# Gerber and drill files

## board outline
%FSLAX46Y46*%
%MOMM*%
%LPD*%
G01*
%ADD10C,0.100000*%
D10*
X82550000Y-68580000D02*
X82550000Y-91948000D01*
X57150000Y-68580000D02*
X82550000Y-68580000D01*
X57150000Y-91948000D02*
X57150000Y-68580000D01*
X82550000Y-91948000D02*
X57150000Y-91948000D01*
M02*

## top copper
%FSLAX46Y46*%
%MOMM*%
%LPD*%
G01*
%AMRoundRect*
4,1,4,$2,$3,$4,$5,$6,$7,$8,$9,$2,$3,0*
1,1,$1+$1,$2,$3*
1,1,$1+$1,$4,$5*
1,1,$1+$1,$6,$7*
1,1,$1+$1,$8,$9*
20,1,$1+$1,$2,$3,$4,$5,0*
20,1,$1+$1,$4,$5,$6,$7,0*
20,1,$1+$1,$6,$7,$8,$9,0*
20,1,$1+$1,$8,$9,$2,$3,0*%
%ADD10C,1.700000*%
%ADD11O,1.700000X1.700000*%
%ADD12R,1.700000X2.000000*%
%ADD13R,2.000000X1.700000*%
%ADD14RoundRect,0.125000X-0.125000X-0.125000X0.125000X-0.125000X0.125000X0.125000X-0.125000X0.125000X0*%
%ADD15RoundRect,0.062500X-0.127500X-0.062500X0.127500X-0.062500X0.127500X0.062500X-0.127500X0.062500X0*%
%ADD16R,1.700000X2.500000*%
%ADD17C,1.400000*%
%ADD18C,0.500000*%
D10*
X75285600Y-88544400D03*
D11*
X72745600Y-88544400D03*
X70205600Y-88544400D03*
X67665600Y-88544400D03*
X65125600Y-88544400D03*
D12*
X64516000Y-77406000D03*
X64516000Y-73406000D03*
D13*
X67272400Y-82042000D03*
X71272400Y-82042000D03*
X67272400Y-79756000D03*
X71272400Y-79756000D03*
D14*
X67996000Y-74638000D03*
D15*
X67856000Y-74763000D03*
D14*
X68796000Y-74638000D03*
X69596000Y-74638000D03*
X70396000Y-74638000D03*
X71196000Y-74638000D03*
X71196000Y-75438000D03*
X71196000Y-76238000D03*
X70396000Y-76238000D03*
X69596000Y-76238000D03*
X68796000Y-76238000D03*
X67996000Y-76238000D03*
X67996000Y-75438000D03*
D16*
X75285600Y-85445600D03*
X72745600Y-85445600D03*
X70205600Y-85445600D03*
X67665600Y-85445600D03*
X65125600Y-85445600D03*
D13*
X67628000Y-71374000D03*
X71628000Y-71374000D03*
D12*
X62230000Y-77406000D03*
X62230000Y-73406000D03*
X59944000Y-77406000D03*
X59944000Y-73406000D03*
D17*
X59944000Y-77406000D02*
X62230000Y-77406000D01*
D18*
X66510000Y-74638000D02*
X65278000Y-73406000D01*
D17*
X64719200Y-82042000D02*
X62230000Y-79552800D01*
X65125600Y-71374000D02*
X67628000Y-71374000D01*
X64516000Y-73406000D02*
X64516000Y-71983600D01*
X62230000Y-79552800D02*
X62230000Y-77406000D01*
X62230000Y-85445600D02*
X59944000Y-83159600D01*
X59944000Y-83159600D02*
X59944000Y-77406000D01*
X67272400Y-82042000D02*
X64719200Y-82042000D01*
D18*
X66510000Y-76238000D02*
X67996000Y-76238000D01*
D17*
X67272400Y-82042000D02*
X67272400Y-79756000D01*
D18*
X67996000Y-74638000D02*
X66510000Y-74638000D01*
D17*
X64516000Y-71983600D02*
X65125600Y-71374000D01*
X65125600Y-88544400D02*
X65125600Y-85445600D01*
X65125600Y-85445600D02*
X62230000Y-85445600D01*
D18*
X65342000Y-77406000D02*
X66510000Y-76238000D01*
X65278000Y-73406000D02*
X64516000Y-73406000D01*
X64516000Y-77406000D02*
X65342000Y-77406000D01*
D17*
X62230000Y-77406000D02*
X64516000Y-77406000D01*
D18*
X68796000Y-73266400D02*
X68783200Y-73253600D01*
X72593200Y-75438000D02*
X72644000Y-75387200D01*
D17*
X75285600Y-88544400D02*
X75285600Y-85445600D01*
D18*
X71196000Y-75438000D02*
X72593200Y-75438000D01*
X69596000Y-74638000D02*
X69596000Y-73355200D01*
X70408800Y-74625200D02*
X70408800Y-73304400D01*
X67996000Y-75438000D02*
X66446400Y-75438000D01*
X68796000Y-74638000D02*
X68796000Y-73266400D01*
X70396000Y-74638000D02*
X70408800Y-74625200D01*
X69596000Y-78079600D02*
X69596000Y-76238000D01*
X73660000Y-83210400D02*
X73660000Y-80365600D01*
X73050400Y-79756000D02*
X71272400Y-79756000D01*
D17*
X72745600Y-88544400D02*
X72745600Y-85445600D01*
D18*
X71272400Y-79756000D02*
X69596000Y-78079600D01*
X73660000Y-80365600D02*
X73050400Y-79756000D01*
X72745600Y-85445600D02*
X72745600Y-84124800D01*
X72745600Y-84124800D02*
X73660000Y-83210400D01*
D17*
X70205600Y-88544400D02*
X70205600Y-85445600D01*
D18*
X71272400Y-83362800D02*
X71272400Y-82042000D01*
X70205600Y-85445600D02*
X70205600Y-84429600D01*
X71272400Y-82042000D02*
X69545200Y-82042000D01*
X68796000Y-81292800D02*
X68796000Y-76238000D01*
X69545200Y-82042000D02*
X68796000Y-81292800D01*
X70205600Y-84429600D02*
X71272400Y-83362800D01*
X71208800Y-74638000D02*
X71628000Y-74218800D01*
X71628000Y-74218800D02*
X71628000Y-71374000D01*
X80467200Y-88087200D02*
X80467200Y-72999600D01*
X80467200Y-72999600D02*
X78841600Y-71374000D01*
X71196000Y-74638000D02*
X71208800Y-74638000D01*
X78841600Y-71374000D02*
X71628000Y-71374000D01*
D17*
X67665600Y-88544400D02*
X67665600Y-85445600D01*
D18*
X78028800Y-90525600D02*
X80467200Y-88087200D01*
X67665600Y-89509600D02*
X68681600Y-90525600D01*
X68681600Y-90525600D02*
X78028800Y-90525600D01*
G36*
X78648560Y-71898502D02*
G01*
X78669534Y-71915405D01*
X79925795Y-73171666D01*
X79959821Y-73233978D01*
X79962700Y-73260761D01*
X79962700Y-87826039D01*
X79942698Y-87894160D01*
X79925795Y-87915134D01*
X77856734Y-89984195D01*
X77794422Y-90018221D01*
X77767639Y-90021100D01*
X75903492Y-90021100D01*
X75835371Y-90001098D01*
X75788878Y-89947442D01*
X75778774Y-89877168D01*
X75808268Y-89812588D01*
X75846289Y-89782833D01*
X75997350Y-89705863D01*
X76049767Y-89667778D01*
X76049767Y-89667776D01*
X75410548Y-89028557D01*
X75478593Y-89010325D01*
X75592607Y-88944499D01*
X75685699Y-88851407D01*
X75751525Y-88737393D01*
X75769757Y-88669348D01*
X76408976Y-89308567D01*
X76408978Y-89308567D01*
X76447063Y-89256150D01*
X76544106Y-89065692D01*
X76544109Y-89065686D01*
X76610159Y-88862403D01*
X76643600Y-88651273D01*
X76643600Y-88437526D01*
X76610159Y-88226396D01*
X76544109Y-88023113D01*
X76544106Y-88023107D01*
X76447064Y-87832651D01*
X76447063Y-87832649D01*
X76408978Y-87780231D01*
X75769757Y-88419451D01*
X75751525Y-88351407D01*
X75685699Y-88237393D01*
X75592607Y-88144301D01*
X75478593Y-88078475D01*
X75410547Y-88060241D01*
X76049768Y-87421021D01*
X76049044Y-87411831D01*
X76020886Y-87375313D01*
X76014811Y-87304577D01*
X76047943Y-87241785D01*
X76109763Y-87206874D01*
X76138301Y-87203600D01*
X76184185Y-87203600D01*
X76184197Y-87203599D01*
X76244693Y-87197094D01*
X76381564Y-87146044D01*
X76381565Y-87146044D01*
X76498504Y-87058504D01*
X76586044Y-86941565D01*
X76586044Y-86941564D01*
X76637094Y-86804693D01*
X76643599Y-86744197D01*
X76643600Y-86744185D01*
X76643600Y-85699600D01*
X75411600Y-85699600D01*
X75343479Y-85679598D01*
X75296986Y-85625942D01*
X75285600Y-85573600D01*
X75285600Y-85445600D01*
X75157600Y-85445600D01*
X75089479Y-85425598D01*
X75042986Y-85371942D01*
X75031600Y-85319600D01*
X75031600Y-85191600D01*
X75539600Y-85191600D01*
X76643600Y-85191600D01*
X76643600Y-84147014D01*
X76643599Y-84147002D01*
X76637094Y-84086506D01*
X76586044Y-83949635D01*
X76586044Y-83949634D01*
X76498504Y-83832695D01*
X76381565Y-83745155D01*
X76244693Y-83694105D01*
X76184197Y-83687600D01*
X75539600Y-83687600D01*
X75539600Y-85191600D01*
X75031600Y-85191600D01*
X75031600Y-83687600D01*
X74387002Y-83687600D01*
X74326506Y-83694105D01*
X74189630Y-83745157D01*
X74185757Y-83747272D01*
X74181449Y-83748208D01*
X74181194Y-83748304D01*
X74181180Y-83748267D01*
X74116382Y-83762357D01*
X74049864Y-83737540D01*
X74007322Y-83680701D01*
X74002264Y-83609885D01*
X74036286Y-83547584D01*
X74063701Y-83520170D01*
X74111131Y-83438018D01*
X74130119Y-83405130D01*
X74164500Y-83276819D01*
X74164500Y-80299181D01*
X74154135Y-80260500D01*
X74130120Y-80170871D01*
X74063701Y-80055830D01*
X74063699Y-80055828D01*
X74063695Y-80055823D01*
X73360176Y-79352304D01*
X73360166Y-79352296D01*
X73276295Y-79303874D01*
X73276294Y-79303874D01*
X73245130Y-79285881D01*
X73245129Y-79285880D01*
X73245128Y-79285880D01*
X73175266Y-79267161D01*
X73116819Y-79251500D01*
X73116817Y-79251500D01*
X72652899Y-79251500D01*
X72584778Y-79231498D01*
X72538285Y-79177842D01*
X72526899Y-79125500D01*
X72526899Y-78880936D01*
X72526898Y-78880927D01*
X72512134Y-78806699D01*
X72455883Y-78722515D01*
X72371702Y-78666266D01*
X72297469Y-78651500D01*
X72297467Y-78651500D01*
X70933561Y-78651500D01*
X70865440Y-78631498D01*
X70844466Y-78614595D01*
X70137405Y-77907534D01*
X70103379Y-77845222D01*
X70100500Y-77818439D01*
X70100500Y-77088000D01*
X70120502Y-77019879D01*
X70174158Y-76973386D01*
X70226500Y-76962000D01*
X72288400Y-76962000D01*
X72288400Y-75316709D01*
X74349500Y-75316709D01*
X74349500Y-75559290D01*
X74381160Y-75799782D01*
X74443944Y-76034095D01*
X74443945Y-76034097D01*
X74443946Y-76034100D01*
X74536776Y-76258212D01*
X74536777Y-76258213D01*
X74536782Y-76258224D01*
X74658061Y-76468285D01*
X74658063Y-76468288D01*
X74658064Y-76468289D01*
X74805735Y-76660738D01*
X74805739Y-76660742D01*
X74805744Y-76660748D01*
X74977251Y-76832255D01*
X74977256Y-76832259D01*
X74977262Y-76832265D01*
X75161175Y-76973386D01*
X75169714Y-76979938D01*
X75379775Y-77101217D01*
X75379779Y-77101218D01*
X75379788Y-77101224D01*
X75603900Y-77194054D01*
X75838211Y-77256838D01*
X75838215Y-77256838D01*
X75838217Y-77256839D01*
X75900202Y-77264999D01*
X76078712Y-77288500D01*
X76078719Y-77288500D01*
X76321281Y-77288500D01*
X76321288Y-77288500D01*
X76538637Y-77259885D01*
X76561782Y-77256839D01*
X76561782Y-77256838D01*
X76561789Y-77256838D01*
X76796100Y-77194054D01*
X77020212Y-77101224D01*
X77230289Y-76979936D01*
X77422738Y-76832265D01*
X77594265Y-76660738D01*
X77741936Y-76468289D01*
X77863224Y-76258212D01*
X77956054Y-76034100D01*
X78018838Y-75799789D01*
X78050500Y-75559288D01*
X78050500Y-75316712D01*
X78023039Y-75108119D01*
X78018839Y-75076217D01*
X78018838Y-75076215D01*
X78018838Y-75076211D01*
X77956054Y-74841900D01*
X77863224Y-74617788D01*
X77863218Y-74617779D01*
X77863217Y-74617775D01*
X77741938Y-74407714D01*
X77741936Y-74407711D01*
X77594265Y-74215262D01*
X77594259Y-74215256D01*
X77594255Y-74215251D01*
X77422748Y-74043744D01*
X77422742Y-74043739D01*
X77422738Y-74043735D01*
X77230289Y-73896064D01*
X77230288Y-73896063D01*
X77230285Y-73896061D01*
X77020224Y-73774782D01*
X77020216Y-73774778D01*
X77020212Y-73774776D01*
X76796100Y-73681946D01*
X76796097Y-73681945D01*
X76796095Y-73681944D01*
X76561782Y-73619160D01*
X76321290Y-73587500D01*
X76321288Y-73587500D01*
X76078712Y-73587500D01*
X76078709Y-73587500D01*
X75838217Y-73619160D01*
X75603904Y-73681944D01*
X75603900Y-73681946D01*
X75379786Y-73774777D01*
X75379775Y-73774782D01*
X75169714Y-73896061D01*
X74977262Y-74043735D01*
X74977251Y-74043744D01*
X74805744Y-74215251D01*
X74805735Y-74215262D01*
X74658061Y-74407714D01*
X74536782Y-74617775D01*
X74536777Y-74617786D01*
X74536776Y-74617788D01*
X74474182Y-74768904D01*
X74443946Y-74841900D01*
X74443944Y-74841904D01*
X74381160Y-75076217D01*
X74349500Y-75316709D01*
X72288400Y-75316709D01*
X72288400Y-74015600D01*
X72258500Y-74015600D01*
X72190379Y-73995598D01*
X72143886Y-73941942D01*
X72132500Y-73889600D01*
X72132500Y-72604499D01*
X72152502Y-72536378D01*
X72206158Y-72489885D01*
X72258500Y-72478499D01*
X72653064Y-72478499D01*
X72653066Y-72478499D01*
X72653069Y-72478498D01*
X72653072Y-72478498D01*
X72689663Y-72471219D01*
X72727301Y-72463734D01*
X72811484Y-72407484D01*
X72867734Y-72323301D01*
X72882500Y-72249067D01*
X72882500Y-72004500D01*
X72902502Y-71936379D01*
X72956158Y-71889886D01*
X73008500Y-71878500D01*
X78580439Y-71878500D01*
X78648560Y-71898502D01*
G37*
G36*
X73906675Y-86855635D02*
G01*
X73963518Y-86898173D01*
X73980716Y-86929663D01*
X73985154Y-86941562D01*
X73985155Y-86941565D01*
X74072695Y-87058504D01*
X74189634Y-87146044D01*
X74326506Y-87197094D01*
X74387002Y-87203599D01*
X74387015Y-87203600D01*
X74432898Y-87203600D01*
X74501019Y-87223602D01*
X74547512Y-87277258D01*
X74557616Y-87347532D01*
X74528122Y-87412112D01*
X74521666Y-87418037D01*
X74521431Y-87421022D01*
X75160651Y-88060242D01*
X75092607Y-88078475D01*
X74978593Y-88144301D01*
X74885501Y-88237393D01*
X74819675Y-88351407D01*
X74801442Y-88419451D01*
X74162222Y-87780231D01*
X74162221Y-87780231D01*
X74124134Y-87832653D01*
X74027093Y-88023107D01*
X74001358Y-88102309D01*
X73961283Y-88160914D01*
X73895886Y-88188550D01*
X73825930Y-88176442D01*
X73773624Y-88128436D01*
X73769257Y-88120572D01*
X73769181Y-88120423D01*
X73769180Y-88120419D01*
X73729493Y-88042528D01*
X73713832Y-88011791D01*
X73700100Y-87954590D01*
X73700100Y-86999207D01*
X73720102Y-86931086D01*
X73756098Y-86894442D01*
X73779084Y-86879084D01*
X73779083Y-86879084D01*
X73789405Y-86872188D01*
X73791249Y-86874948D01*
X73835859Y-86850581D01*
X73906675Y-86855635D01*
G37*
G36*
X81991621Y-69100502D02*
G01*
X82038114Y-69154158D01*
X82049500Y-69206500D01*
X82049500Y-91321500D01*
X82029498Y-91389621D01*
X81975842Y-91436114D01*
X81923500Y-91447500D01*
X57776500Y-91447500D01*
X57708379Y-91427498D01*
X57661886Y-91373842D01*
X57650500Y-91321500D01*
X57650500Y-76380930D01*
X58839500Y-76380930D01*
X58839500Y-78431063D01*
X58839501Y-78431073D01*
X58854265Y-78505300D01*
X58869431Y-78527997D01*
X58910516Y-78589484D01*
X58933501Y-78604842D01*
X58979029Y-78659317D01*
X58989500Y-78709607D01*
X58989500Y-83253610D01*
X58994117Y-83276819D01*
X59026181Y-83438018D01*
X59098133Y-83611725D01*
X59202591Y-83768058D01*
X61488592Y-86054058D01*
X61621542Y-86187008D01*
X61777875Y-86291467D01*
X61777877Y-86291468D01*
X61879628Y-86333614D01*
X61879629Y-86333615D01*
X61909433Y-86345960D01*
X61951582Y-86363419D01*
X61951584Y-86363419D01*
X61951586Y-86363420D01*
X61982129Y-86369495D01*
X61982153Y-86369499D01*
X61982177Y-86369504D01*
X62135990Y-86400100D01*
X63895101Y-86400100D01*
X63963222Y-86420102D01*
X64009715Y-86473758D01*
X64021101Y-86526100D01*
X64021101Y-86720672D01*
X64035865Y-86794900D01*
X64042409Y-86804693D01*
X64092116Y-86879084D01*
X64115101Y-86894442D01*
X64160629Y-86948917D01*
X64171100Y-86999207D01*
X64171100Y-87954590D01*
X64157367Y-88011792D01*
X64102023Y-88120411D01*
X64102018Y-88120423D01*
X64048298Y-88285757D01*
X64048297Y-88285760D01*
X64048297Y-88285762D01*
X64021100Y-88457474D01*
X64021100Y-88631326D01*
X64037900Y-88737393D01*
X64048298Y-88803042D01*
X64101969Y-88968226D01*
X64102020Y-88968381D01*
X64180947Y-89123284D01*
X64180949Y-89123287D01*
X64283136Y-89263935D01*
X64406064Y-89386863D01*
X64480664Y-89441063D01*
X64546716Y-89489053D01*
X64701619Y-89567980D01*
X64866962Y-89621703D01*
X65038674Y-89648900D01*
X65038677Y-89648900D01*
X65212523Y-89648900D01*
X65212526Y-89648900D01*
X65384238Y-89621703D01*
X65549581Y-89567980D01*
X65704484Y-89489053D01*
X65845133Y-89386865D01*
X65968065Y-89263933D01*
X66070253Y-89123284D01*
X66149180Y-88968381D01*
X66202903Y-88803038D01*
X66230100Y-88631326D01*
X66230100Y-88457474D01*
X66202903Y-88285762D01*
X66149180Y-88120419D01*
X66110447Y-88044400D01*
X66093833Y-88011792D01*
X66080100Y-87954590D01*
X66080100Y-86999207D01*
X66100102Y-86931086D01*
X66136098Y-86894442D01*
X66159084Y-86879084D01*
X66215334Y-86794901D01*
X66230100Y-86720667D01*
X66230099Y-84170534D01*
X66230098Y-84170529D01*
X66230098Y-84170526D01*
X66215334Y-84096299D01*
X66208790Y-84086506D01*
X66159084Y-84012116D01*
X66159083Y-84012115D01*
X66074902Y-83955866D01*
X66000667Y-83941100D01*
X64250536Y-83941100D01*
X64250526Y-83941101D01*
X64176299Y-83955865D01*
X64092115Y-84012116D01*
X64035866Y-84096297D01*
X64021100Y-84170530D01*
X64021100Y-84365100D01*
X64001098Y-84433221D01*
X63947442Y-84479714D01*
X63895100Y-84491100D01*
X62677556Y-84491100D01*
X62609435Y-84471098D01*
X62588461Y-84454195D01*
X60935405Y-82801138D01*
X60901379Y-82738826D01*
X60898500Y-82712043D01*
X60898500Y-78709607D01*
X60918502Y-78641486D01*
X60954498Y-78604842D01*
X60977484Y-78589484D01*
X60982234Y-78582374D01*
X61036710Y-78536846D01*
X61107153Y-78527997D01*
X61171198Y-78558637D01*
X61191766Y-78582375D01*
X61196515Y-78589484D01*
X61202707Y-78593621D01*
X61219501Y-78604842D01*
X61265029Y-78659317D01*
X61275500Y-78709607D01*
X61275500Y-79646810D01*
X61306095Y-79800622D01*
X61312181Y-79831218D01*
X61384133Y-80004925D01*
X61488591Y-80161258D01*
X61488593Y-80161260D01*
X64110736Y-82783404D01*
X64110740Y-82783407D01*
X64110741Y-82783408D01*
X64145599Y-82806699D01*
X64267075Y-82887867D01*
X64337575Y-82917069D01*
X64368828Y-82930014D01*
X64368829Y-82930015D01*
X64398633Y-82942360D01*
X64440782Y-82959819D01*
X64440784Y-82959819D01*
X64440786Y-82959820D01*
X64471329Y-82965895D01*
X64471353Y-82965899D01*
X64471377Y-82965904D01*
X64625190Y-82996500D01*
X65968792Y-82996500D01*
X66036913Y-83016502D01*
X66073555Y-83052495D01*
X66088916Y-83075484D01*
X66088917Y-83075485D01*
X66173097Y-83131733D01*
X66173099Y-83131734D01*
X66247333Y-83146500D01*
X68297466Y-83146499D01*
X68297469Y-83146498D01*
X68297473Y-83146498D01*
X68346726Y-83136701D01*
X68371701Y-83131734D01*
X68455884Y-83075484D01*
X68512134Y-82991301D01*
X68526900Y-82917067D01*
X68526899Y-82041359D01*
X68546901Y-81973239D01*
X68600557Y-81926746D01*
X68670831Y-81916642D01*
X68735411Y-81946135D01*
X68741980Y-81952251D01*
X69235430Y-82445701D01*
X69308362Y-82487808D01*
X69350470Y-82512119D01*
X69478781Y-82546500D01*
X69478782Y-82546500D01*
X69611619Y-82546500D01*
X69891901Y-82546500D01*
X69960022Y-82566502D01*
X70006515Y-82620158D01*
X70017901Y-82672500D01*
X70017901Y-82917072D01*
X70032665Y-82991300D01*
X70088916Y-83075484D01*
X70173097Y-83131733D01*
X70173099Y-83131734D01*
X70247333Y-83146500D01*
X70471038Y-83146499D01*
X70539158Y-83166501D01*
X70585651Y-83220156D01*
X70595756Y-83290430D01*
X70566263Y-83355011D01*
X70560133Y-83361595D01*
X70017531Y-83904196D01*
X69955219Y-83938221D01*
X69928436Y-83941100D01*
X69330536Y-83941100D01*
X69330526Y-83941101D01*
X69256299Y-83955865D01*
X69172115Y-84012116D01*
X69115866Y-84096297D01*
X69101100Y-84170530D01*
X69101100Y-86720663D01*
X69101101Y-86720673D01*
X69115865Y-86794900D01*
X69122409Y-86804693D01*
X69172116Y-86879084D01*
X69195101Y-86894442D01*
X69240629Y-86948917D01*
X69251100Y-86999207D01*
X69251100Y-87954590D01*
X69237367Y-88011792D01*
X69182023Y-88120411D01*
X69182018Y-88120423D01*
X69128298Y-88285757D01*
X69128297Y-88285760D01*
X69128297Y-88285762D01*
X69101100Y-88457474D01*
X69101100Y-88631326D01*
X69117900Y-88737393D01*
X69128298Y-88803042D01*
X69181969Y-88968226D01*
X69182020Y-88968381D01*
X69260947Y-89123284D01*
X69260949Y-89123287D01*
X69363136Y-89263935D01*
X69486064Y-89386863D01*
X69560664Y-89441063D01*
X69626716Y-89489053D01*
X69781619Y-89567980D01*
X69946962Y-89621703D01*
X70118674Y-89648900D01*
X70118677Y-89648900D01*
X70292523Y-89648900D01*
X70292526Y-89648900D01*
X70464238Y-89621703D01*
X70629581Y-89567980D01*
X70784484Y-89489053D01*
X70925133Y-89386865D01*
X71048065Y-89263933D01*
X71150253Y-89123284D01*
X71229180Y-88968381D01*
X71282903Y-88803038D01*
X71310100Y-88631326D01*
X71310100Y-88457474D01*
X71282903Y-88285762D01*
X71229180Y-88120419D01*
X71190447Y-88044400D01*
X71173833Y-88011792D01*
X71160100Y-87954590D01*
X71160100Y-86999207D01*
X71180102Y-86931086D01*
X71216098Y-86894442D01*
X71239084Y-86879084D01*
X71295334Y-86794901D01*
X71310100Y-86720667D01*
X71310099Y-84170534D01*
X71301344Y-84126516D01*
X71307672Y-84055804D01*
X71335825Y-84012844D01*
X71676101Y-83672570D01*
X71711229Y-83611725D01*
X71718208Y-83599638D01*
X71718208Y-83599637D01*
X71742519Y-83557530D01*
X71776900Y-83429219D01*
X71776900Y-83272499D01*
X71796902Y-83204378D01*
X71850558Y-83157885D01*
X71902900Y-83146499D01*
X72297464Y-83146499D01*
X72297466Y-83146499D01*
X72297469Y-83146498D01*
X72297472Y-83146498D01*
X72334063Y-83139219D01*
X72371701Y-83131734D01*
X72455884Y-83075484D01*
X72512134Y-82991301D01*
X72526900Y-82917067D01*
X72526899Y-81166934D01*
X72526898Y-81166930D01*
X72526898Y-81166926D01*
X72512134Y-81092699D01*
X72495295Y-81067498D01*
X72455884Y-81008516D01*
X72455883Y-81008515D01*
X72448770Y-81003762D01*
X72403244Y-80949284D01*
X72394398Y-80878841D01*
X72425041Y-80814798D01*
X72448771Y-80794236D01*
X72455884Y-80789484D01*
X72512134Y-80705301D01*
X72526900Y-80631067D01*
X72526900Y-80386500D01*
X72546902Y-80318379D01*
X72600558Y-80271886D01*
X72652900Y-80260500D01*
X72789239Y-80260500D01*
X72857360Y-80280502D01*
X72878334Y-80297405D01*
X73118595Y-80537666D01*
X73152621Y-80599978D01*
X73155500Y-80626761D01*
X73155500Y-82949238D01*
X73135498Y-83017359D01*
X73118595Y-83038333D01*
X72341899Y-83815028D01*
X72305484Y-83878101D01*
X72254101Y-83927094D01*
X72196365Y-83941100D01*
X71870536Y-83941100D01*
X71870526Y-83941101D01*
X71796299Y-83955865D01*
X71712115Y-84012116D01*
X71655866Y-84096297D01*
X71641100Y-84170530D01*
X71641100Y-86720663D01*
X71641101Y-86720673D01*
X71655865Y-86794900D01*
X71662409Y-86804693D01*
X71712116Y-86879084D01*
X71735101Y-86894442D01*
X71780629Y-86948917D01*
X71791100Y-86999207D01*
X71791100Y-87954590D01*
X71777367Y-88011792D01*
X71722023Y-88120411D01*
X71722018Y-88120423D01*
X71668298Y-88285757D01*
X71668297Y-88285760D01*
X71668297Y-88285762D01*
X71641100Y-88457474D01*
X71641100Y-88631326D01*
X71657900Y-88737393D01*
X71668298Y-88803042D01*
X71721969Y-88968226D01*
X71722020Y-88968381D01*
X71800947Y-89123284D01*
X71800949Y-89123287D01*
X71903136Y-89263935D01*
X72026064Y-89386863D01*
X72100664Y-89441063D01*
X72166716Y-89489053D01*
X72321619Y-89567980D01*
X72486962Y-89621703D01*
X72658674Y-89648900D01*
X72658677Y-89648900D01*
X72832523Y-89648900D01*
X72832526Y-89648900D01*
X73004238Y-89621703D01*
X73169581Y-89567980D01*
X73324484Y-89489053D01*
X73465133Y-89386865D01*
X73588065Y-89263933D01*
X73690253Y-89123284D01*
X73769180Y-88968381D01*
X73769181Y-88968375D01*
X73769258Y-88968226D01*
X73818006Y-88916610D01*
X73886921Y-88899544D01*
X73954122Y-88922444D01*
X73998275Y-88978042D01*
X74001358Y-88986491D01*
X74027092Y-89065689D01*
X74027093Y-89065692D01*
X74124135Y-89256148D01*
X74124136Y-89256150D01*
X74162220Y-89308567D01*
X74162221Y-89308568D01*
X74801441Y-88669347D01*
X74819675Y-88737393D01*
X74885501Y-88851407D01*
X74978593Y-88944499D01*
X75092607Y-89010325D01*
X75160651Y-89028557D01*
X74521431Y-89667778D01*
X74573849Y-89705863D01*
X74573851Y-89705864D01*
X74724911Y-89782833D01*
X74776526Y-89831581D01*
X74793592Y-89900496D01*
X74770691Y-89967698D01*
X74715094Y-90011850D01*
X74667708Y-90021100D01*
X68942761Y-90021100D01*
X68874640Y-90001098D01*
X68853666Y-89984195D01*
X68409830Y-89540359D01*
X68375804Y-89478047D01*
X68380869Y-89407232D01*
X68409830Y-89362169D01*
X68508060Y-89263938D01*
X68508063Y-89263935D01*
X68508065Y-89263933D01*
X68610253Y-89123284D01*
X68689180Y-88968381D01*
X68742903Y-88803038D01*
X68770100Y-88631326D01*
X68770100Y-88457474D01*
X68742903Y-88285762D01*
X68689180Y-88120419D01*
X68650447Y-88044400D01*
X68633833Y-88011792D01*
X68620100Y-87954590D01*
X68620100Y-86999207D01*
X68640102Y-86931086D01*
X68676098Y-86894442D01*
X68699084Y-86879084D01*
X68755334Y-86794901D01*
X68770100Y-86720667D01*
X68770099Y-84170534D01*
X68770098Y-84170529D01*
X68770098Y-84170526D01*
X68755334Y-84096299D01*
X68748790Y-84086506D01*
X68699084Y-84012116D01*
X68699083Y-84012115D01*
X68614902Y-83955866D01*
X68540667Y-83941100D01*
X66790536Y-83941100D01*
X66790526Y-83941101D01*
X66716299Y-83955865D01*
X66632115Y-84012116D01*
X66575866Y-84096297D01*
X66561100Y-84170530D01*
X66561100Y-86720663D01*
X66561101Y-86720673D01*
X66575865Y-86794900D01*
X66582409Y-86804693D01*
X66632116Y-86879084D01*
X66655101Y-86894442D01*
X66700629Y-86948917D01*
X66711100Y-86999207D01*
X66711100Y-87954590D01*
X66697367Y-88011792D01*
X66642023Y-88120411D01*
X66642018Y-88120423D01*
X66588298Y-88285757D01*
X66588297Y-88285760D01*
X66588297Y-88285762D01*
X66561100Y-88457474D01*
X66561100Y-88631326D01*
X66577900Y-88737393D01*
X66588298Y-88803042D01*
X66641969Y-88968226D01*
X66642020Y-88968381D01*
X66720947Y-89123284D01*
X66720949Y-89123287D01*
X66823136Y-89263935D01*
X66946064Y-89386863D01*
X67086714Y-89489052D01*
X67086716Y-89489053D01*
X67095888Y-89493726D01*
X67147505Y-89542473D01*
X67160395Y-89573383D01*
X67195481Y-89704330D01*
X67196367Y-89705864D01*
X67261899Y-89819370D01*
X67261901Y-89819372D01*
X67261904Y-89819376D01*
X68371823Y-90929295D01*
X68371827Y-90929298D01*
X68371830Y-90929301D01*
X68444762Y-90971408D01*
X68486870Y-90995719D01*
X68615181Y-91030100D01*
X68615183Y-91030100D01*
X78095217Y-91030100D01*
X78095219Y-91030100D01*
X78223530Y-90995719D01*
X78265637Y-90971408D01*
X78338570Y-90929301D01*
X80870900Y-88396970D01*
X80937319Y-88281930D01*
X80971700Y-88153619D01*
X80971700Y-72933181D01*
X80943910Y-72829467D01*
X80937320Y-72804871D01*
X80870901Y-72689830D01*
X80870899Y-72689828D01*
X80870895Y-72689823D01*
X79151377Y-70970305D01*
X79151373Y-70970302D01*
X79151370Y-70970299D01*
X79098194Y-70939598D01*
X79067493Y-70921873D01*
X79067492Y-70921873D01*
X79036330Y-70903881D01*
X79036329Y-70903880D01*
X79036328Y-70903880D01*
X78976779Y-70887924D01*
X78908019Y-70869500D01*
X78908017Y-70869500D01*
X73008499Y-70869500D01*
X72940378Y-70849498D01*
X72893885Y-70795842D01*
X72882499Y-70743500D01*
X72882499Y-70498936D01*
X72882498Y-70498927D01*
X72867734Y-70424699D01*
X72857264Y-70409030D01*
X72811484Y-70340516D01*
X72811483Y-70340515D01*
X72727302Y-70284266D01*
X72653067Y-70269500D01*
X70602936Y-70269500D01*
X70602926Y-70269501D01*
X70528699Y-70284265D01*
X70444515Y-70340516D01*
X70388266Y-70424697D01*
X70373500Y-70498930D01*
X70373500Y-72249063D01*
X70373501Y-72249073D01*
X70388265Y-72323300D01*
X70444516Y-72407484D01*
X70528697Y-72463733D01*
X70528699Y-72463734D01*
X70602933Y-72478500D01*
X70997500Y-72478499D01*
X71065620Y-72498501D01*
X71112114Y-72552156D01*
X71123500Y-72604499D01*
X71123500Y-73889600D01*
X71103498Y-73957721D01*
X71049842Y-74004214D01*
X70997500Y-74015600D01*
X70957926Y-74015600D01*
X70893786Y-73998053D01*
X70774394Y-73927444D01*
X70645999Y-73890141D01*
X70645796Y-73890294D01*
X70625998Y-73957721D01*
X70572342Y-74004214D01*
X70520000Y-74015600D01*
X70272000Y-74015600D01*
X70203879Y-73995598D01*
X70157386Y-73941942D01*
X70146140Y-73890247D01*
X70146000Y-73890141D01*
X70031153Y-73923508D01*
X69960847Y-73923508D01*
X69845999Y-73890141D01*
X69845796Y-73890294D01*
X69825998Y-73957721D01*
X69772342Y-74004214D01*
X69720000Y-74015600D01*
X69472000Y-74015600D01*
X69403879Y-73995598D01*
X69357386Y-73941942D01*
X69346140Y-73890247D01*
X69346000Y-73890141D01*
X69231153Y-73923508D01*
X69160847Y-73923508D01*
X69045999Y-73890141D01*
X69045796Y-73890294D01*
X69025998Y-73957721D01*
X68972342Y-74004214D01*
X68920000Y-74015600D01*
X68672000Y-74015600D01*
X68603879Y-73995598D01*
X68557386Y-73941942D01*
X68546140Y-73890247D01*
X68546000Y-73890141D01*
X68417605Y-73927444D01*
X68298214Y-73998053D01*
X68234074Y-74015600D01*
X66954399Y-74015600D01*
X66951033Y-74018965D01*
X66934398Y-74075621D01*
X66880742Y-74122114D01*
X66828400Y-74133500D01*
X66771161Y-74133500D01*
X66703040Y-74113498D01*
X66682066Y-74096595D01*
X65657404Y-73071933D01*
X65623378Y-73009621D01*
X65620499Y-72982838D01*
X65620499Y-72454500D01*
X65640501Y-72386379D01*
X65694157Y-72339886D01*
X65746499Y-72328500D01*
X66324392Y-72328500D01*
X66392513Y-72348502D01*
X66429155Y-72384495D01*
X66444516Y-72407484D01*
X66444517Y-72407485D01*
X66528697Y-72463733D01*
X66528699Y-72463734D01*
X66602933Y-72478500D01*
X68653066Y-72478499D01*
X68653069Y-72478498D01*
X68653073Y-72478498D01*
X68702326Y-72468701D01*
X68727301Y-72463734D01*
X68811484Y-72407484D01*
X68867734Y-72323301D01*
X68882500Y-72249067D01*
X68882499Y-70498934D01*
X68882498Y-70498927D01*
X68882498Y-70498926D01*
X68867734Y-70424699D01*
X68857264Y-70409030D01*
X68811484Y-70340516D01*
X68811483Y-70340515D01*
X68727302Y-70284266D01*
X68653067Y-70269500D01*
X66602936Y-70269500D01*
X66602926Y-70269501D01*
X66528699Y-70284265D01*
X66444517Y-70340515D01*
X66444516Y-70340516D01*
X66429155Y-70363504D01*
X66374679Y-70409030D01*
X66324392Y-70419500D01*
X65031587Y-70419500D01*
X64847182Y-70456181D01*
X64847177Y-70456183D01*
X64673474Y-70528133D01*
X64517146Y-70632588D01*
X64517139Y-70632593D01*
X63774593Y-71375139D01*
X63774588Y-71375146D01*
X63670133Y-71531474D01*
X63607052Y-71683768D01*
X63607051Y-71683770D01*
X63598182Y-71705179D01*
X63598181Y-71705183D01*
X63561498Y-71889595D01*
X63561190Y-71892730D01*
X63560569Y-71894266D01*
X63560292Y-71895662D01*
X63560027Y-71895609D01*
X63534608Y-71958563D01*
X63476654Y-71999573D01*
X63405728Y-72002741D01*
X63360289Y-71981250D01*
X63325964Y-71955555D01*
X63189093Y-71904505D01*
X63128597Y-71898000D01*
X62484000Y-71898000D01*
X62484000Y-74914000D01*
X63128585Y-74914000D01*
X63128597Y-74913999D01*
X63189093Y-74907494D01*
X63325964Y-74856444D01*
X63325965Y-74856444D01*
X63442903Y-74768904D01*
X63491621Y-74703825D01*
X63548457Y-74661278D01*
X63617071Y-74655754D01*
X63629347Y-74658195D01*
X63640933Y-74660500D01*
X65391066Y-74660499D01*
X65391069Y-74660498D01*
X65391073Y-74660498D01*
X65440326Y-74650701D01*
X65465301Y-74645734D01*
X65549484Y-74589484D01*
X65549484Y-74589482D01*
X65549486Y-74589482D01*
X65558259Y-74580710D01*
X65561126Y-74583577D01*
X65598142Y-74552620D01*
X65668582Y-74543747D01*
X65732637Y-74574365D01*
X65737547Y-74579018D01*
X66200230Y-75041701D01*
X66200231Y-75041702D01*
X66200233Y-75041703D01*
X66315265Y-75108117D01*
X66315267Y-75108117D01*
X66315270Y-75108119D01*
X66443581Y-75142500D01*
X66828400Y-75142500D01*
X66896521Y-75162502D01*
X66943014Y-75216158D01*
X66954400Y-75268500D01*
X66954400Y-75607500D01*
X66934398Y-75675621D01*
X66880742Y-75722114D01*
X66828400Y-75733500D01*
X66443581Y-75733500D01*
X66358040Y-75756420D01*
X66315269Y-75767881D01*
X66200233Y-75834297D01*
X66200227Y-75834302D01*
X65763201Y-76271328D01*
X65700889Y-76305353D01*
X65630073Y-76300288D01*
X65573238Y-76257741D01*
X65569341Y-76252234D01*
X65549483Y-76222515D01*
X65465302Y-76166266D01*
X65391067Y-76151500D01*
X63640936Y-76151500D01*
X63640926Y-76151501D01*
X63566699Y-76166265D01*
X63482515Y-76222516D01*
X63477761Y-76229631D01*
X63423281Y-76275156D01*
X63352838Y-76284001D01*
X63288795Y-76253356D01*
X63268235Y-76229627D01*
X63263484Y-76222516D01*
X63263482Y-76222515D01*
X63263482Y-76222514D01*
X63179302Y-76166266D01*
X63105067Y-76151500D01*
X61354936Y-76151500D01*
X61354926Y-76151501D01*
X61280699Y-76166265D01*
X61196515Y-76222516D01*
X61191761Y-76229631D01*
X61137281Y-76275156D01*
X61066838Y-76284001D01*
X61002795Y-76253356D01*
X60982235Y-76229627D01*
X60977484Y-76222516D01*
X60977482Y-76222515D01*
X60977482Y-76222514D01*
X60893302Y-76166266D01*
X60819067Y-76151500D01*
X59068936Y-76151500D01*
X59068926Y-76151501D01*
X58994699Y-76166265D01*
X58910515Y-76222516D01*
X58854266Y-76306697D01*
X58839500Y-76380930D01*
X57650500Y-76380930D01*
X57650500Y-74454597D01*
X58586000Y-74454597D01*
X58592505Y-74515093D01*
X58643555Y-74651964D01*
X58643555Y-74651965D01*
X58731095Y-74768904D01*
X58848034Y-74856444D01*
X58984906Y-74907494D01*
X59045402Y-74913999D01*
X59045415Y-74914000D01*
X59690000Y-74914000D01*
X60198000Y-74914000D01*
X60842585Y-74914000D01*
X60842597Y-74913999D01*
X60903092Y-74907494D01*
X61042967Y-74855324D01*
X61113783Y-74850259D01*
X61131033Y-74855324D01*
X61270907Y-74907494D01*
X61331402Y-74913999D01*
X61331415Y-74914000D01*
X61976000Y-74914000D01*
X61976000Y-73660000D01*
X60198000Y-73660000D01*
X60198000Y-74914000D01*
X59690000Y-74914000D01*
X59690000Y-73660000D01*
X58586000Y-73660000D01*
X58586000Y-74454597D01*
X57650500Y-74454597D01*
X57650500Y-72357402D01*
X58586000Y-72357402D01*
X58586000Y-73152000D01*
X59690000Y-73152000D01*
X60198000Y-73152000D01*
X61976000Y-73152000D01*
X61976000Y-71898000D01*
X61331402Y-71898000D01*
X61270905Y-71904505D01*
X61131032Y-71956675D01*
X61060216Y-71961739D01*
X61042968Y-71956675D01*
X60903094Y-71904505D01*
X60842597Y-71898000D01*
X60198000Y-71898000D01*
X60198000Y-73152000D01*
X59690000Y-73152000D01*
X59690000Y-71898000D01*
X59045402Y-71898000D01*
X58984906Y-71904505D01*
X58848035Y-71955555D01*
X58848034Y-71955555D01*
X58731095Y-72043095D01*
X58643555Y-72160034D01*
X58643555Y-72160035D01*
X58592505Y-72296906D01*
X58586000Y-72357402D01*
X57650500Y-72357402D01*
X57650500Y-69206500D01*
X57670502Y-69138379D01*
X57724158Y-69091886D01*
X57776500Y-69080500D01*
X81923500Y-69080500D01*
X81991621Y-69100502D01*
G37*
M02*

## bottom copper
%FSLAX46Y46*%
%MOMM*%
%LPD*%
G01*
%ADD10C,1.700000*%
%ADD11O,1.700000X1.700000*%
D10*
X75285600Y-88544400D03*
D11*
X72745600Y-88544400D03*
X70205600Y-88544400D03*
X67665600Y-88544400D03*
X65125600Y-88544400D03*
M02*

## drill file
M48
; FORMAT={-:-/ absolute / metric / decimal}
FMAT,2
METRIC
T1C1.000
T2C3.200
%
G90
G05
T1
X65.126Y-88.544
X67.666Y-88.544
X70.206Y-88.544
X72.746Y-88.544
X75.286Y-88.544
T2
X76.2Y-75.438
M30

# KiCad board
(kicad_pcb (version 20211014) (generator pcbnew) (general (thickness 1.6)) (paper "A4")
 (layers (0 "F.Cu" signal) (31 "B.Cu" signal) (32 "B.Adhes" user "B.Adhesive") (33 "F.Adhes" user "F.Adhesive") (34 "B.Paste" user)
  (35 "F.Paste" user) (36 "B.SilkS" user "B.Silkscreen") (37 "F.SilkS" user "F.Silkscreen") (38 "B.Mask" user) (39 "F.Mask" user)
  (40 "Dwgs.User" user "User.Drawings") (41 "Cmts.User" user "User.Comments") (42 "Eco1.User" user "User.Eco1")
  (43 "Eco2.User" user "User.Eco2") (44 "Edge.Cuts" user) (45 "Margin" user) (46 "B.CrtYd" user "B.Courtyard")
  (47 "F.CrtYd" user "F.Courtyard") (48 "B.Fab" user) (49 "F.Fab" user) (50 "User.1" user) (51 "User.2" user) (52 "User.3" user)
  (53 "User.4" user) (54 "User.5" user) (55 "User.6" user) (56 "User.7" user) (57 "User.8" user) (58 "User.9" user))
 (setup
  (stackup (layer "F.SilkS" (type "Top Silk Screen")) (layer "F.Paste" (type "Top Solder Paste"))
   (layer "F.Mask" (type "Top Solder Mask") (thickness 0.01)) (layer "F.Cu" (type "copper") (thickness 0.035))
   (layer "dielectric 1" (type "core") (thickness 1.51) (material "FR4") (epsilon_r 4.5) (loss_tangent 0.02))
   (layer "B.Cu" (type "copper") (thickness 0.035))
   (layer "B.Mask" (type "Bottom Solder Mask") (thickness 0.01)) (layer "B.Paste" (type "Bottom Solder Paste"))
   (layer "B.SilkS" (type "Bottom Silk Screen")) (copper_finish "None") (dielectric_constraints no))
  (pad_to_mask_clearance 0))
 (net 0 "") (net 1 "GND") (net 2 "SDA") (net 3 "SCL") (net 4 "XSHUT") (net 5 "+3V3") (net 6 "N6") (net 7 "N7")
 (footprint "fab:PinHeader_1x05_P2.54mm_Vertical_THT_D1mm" (layer "F.Cu") (at 75.2856 88.5444 -90)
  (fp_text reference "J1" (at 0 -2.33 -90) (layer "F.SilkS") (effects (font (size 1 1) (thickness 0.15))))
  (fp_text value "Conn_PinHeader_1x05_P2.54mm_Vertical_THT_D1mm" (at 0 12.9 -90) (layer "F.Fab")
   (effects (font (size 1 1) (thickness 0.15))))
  (pad "1" thru_hole circle locked (at 0 0 270) (size 1.7 1.7) (drill 1) (layers *.Cu *.Mask) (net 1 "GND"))
  (pad "2" thru_hole oval locked (at 0 2.54 270) (size 1.7 1.7) (drill 1) (layers *.Cu *.Mask) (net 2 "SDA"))
  (pad "3" thru_hole oval locked (at 0 5.08 270) (size 1.7 1.7) (drill 1) (layers *.Cu *.Mask) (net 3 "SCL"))
  (pad "4" thru_hole oval locked (at 0 7.62 270) (size 1.7 1.7) (drill 1) (layers *.Cu *.Mask) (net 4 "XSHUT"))
  (pad "5" thru_hole oval locked (at 0 10.16 270) (size 1.7 1.7) (drill 1) (layers *.Cu *.Mask) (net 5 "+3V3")))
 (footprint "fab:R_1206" (layer "F.Cu") (at 64.516 75.406 90)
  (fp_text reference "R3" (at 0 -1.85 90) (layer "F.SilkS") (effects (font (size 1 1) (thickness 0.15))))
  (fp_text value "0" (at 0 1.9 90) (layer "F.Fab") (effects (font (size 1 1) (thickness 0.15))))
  (pad "1" smd rect locked (at -2 0 90) (size 2 1.7) (layers "F.Cu" "F.Paste" "F.Mask") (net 5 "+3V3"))
  (pad "2" smd rect locked (at 2 0 90) (size 2 1.7) (layers "F.Cu" "F.Paste" "F.Mask") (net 5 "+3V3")))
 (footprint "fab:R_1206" (layer "F.Cu") (at 69.2724 82.042)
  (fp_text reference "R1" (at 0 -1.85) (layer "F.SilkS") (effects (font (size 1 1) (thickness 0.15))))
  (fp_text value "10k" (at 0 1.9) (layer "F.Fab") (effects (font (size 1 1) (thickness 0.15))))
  (pad "1" smd rect locked (at -2 0) (size 2 1.7) (layers "F.Cu" "F.Paste" "F.Mask") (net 5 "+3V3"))
  (pad "2" smd rect locked (at 2 0) (size 2 1.7) (layers "F.Cu" "F.Paste" "F.Mask") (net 3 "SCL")))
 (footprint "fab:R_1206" (layer "F.Cu") (at 69.2724 79.756)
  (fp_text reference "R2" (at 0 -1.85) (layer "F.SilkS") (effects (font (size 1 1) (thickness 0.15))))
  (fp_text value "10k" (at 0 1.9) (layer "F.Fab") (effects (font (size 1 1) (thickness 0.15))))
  (pad "1" smd rect locked (at -2 0) (size 2 1.7) (layers "F.Cu" "F.Paste" "F.Mask") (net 5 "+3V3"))
  (pad "2" smd rect locked (at 2 0) (size 2 1.7) (layers "F.Cu" "F.Paste" "F.Mask") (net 2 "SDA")))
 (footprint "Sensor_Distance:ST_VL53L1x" (layer "F.Cu") (at 69.596 75.438)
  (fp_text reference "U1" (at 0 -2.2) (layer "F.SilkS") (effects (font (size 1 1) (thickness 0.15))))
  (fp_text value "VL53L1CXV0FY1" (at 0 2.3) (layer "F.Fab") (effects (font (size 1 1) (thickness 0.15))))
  (pad "1" smd roundrect (at -1.6 -0.8) (size 0.5 0.5) (layers "F.Cu" "F.Paste" "F.Mask") (roundrect_rratio 0.25) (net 5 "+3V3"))
  (pad "1" smd roundrect (at -1.74 -0.675) (size 0.38 0.25) (layers "F.Cu" "F.Paste" "F.Mask") (roundrect_rratio 0.25) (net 5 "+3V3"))
  (pad "2" smd roundrect (at -0.8 -0.8) (size 0.5 0.5) (layers "F.Cu" "F.Paste" "F.Mask") (roundrect_rratio 0.25) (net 1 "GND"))
  (pad "3" smd roundrect (at 0 -0.8) (size 0.5 0.5) (layers "F.Cu" "F.Paste" "F.Mask") (roundrect_rratio 0.25) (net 1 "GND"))
  (pad "4" smd roundrect (at 0.8 -0.8) (size 0.5 0.5) (layers "F.Cu" "F.Paste" "F.Mask") (roundrect_rratio 0.25) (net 1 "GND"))
  (pad "5" smd roundrect (at 1.6 -0.8) (size 0.5 0.5) (layers "F.Cu" "F.Paste" "F.Mask") (roundrect_rratio 0.25) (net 4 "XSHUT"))
  (pad "6" smd roundrect (at 1.6 0) (size 0.5 0.5) (layers "F.Cu" "F.Paste" "F.Mask") (roundrect_rratio 0.25) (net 1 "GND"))
  (pad "7" smd roundrect (at 1.6 0.8) (size 0.5 0.5) (layers "F.Cu" "F.Paste" "F.Mask") (roundrect_rratio 0.25) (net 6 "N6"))
  (pad "8" smd roundrect (at 0.8 0.8) (size 0.5 0.5) (layers "F.Cu" "F.Paste" "F.Mask") (roundrect_rratio 0.25) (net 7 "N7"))
  (pad "9" smd roundrect (at 0 0.8) (size 0.5 0.5) (layers "F.Cu" "F.Paste" "F.Mask") (roundrect_rratio 0.25) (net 2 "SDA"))
  (pad "10" smd roundrect (at -0.8 0.8) (size 0.5 0.5) (layers "F.Cu" "F.Paste" "F.Mask") (roundrect_rratio 0.25) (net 3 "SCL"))
  (pad "11" smd roundrect (at -1.6 0.8) (size 0.5 0.5) (layers "F.Cu" "F.Paste" "F.Mask") (roundrect_rratio 0.25) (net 5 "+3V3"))
  (pad "12" smd roundrect (at -1.6 0) (size 0.5 0.5) (layers "F.Cu" "F.Paste" "F.Mask") (roundrect_rratio 0.25) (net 1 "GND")))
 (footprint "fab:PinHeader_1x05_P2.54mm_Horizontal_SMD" (layer "F.Cu") (at 75.2856 85.4456 -90)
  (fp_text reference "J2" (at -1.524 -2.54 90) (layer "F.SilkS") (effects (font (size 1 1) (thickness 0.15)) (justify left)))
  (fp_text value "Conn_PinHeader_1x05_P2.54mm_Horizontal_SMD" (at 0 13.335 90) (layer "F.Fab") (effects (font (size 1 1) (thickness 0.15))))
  (pad "1" smd rect locked (at 0 0 270) (size 2.5 1.7) (layers "F.Cu" "F.Paste" "F.Mask") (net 1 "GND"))
  (pad "2" smd rect locked (at 0 2.54 270) (size 2.5 1.7) (layers "F.Cu" "F.Paste" "F.Mask") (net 2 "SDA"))
  (pad "3" smd rect locked (at 0 5.08 270) (size 2.5 1.7) (layers "F.Cu" "F.Paste" "F.Mask") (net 3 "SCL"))
  (pad "4" smd rect locked (at 0 7.62 270) (size 2.5 1.7) (layers "F.Cu" "F.Paste" "F.Mask") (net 4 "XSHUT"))
  (pad "5" smd rect locked (at 0 10.16 270) (size 2.5 1.7) (layers "F.Cu" "F.Paste" "F.Mask") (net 5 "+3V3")))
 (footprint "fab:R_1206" (layer "F.Cu") (at 69.628 71.374)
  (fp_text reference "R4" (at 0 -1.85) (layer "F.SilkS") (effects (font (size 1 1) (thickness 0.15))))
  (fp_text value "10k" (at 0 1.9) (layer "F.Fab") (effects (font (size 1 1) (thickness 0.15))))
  (pad "1" smd rect locked (at -2 0) (size 2 1.7) (layers "F.Cu" "F.Paste" "F.Mask") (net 5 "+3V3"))
  (pad "2" smd rect locked (at 2 0) (size 2 1.7) (layers "F.Cu" "F.Paste" "F.Mask") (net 4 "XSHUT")))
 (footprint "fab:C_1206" (layer "F.Cu") (at 62.23 75.406 90)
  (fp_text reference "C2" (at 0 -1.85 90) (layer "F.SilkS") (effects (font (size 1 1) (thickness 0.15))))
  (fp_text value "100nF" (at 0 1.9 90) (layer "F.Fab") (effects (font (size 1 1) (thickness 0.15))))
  (pad "1" smd rect (at -2 0 90) (size 2 1.7) (layers "F.Cu" "F.Paste" "F.Mask") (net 5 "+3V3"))
  (pad "2" smd rect (at 2 0 90) (size 2 1.7) (layers "F.Cu" "F.Paste" "F.Mask") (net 1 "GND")))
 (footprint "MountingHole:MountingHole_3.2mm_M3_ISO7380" (layer "F.Cu") (at 76.2 75.438)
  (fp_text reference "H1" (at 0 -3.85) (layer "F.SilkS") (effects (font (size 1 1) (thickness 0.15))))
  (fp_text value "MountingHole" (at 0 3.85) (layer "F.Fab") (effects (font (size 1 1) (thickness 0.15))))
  (pad "" np_thru_hole circle (at 0 0) (size 3.2 3.2) (drill 3.2) (layers *.Cu *.Mask)))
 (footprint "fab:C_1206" (layer "F.Cu") (at 59.944 75.406 90)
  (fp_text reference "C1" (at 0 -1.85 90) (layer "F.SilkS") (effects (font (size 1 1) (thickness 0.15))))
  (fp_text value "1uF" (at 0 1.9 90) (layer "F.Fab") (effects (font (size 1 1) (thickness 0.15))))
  (pad "1" smd rect (at -2 0 90) (size 2 1.7) (layers "F.Cu" "F.Paste" "F.Mask") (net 5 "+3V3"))
  (pad "2" smd rect (at 2 0 90) (size 2 1.7) (layers "F.Cu" "F.Paste" "F.Mask") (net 1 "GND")))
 (gr_line (start 82.55 68.58) (end 82.55 91.948) (layer "Edge.Cuts") (width 0.1))
 (gr_line (start 57.15 68.58) (end 82.55 68.58) (layer "Edge.Cuts") (width 0.1))
 (gr_line (start 57.15 91.948) (end 57.15 68.58) (layer "Edge.Cuts") (width 0.1))
 (gr_line (start 82.55 91.948) (end 57.15 91.948) (layer "Edge.Cuts") (width 0.1))
 (segment (start 59.944 77.406) (end 62.23 77.406) (width 1.4) (layer "F.Cu") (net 5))
 (segment (start 66.51 74.638) (end 65.278 73.406) (width 0.5) (layer "F.Cu") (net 5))
 (segment (start 64.7192 82.042) (end 62.23 79.5528) (width 1.4) (layer "F.Cu") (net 5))
 (segment (start 65.1256 71.374) (end 67.628 71.374) (width 1.4) (layer "F.Cu") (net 5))
 (segment (start 64.516 73.406) (end 64.516 71.9836) (width 1.4) (layer "F.Cu") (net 5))
 (segment (start 62.23 79.5528) (end 62.23 77.406) (width 1.4) (layer "F.Cu") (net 5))
 (segment (start 62.23 85.4456) (end 59.944 83.1596) (width 1.4) (layer "F.Cu") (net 5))
 (segment (start 59.944 83.1596) (end 59.944 77.406) (width 1.4) (layer "F.Cu") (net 5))
 (segment (start 67.2724 82.042) (end 64.7192 82.042) (width 1.4) (layer "F.Cu") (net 5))
 (segment (start 66.51 76.238) (end 67.996 76.238) (width 0.5) (layer "F.Cu") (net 5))
 (segment (start 67.2724 82.042) (end 67.2724 79.756) (width 1.4) (layer "F.Cu") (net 5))
 (segment (start 67.996 74.638) (end 66.51 74.638) (width 0.5) (layer "F.Cu") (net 5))
 (segment (start 64.516 71.9836) (end 65.1256 71.374) (width 1.4) (layer "F.Cu") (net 5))
 (segment (start 65.1256 88.5444) (end 65.1256 85.4456) (width 1.4) (layer "F.Cu") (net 5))
 (segment (start 65.1256 85.4456) (end 62.23 85.4456) (width 1.4) (layer "F.Cu") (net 5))
 (segment (start 65.342 77.406) (end 66.51 76.238) (width 0.5) (layer "F.Cu") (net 5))
 (segment (start 65.278 73.406) (end 64.516 73.406) (width 0.5) (layer "F.Cu") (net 5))
 (segment (start 64.516 77.406) (end 65.342 77.406) (width 0.5) (layer "F.Cu") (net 5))
 (segment (start 62.23 77.406) (end 64.516 77.406) (width 1.4) (layer "F.Cu") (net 5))
 (segment (start 68.796 73.2664) (end 68.7832 73.2536) (width 0.5) (layer "F.Cu") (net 1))
 (segment (start 72.5932 75.438) (end 72.644 75.3872) (width 0.5) (layer "F.Cu") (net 1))
 (segment (start 75.2856 88.5444) (end 75.2856 85.4456) (width 1.4) (layer "F.Cu") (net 1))
 (segment (start 71.196 75.438) (end 72.5932 75.438) (width 0.5) (layer "F.Cu") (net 1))
 (segment (start 69.596 74.638) (end 69.596 73.3552) (width 0.5) (layer "F.Cu") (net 1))
 (segment (start 70.4088 74.6252) (end 70.4088 73.3044) (width 0.5) (layer "F.Cu") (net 1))
 (segment (start 67.996 75.438) (end 66.4464 75.438) (width 0.5) (layer "F.Cu") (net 1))
 (segment (start 68.796 74.638) (end 68.796 73.2664) (width 0.5) (layer "F.Cu") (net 1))
 (segment (start 70.396 74.638) (end 70.4088 74.6252) (width 0.5) (layer "F.Cu") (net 1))
 (segment (start 69.596 78.0796) (end 69.596 76.238) (width 0.5) (layer "F.Cu") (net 2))
 (segment (start 73.66 83.2104) (end 73.66 80.3656) (width 0.5) (layer "F.Cu") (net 2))
 (segment (start 73.0504 79.756) (end 71.2724 79.756) (width 0.5) (layer "F.Cu") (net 2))
 (segment (start 72.7456 88.5444) (end 72.7456 85.4456) (width 1.4) (layer "F.Cu") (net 2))
 (segment (start 71.2724 79.756) (end 69.596 78.0796) (width 0.5) (layer "F.Cu") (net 2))
 (segment (start 73.66 80.3656) (end 73.0504 79.756) (width 0.5) (layer "F.Cu") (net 2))
 (segment (start 72.7456 85.4456) (end 72.7456 84.1248) (width 0.5) (layer "F.Cu") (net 2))
 (segment (start 72.7456 84.1248) (end 73.66 83.2104) (width 0.5) (layer "F.Cu") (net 2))
 (segment (start 70.2056 88.5444) (end 70.2056 85.4456) (width 1.4) (layer "F.Cu") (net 3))
 (segment (start 71.2724 83.3628) (end 71.2724 82.042) (width 0.5) (layer "F.Cu") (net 3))
 (segment (start 70.2056 85.4456) (end 70.2056 84.4296) (width 0.5) (layer "F.Cu") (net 3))
 (segment (start 71.2724 82.042) (end 69.5452 82.042) (width 0.5) (layer "F.Cu") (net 3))
 (segment (start 68.796 81.2928) (end 68.796 76.238) (width 0.5) (layer "F.Cu") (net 3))
 (segment (start 69.5452 82.042) (end 68.796 81.2928) (width 0.5) (layer "F.Cu") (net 3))
 (segment (start 70.2056 84.4296) (end 71.2724 83.3628) (width 0.5) (layer "F.Cu") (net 3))
 (segment (start 71.2088 74.638) (end 71.628 74.2188) (width 0.5) (layer "F.Cu") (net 4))
 (segment (start 71.628 74.2188) (end 71.628 71.374) (width 0.5) (layer "F.Cu") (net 4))
 (segment (start 80.4672 88.0872) (end 80.4672 72.9996) (width 0.5) (layer "F.Cu") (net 4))
 (segment (start 80.4672 72.9996) (end 78.8416 71.374) (width 0.5) (layer "F.Cu") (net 4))
 (segment (start 71.196 74.638) (end 71.2088 74.638) (width 0.5) (layer "F.Cu") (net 4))
 (segment (start 78.8416 71.374) (end 71.628 71.374) (width 0.5) (layer "F.Cu") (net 4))
 (segment (start 67.6656 88.5444) (end 67.6656 85.4456) (width 1.4) (layer "F.Cu") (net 4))
 (segment (start 78.0288 90.5256) (end 80.4672 88.0872) (width 0.5) (layer "F.Cu") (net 4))
 (segment (start 67.6656 89.5096) (end 68.6816 90.5256) (width 0.5) (layer "F.Cu") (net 4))
 (segment (start 68.6816 90.5256) (end 78.0288 90.5256) (width 0.5) (layer "F.Cu") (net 4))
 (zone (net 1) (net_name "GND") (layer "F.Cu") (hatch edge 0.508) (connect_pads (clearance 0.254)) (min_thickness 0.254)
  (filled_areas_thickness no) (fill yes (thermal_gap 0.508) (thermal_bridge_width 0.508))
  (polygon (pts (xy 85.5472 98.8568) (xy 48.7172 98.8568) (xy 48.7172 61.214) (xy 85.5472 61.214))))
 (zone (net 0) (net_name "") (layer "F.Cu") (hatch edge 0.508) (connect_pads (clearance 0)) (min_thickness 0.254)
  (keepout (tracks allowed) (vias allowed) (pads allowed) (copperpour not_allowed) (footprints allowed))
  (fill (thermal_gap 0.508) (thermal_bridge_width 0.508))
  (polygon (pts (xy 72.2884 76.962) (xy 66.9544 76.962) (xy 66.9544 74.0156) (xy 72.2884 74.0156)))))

